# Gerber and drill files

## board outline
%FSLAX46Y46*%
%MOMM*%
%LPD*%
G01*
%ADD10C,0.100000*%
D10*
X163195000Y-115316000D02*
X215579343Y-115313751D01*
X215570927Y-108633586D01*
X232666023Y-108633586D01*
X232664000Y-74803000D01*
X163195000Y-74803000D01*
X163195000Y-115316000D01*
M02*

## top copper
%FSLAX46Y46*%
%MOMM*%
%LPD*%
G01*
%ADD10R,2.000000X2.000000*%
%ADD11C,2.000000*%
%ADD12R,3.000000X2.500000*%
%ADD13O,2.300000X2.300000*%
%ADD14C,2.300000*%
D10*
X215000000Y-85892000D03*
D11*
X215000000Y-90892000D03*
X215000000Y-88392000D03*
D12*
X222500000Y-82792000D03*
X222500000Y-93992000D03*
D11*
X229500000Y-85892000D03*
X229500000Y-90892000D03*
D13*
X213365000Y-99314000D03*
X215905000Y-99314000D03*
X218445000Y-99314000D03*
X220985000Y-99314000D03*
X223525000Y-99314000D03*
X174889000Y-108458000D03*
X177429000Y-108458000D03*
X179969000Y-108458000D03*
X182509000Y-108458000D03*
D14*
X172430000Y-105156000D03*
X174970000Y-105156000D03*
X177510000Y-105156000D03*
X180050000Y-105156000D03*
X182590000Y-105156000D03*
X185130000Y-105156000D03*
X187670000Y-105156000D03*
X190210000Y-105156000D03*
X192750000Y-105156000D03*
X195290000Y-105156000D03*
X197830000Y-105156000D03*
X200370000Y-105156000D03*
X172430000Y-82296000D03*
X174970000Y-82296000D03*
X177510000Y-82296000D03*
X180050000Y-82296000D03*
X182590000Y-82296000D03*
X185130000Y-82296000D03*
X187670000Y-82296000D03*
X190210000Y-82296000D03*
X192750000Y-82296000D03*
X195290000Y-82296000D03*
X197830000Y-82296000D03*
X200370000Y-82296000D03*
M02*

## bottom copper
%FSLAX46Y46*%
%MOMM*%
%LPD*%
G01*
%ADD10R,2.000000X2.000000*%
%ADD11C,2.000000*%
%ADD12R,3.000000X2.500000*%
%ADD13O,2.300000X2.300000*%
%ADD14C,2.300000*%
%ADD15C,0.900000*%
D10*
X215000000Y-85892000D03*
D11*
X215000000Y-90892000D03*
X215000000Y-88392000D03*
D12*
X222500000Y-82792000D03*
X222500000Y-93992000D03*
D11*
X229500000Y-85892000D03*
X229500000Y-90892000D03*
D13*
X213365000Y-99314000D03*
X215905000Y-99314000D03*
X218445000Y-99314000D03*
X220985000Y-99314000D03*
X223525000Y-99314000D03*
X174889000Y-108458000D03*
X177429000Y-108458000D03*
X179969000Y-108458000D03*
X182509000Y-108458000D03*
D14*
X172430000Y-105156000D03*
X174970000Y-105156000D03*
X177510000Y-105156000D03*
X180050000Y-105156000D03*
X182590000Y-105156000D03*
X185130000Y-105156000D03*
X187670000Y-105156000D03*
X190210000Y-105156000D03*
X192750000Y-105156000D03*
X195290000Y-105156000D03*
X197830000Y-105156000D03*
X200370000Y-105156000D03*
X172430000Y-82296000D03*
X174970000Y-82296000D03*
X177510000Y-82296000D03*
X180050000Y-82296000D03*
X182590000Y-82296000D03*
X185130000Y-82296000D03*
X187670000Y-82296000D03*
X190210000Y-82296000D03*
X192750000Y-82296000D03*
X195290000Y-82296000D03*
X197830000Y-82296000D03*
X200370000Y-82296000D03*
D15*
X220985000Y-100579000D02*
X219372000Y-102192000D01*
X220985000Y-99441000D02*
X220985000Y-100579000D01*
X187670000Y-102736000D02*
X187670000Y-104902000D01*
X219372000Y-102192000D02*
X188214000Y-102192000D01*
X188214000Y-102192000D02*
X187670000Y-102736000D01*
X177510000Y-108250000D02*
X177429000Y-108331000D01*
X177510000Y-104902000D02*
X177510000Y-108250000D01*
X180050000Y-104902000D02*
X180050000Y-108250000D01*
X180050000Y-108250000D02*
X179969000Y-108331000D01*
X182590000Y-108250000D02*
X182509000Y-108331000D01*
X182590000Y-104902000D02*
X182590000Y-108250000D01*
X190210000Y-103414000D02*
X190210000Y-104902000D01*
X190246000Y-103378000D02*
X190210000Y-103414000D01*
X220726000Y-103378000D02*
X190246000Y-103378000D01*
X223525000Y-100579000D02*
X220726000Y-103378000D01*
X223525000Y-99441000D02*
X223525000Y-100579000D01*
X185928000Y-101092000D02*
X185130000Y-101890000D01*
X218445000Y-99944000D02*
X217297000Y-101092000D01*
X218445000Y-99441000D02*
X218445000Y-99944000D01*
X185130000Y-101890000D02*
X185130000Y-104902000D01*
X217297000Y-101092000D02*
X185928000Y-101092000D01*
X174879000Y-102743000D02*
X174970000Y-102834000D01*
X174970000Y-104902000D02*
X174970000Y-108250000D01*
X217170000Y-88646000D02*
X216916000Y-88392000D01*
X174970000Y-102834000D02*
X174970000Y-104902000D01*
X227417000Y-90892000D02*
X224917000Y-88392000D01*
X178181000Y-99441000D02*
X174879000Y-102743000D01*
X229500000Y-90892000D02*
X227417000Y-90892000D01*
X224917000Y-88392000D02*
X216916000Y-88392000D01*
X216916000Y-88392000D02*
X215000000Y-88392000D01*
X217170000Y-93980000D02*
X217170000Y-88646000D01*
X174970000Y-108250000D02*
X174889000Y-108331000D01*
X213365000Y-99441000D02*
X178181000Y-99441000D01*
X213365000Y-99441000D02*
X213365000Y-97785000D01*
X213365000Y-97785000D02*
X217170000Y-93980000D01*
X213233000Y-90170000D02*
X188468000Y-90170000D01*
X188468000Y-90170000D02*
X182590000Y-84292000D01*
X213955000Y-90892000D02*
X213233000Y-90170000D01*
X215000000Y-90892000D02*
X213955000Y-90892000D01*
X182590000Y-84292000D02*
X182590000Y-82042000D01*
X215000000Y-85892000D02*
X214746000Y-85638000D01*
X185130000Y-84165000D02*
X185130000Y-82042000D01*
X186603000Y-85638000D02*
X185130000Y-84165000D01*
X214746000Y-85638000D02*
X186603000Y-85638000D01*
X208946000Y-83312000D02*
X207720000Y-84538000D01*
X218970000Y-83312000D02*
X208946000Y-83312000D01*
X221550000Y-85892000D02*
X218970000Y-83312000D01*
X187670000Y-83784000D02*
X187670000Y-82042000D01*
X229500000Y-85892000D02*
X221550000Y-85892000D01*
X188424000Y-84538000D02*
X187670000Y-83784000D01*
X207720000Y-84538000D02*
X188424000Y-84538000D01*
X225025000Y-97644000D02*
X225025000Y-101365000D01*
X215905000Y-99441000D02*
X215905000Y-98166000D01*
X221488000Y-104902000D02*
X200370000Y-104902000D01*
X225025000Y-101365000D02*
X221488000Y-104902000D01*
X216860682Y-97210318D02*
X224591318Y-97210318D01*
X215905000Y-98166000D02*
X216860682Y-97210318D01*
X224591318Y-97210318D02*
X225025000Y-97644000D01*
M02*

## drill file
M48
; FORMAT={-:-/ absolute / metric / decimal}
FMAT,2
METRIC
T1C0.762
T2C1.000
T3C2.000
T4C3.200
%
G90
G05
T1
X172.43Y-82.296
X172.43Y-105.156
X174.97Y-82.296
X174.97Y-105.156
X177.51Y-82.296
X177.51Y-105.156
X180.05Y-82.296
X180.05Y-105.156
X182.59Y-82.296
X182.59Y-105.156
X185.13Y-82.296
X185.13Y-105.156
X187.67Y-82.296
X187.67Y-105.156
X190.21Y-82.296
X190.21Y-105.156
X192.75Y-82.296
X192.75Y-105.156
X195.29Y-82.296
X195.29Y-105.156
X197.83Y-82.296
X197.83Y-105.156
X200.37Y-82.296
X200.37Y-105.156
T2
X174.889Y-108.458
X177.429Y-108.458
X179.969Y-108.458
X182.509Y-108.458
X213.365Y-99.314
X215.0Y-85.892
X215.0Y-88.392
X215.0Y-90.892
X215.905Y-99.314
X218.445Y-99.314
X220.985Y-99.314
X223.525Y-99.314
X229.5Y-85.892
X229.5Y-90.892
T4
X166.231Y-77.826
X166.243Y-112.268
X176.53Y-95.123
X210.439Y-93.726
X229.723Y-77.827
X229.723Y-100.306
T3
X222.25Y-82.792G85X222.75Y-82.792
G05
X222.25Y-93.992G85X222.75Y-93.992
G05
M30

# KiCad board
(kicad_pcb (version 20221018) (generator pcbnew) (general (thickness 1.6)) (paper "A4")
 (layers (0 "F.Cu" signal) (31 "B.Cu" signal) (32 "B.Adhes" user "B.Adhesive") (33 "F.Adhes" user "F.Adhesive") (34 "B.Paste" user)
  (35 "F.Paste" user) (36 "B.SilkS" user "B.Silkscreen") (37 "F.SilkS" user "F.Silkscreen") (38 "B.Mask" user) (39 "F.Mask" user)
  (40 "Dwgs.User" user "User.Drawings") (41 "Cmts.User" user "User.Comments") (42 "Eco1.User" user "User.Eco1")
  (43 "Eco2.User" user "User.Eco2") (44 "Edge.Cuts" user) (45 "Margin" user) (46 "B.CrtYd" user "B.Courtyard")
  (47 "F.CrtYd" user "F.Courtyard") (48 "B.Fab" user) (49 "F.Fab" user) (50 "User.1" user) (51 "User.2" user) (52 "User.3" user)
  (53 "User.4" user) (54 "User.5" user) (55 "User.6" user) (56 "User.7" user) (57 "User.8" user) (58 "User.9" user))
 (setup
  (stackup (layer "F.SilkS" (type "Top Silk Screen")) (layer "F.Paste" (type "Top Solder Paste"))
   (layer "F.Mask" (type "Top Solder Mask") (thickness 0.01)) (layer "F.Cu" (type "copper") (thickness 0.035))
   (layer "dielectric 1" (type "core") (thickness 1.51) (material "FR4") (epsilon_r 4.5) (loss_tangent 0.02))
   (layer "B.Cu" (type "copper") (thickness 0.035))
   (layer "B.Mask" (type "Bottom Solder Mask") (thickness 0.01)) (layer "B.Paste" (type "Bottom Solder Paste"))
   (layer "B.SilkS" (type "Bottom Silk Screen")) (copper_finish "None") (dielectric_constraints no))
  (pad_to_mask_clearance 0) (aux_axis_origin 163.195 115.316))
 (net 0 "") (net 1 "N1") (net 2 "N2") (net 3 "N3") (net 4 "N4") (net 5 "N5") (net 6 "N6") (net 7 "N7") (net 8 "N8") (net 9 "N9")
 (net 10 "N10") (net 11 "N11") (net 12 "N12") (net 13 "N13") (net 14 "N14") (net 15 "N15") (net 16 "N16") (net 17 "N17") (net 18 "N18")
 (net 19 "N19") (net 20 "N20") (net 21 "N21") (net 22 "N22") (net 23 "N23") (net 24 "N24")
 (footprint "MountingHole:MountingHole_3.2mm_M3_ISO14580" (layer "F.Cu") (at 210.439 93.726)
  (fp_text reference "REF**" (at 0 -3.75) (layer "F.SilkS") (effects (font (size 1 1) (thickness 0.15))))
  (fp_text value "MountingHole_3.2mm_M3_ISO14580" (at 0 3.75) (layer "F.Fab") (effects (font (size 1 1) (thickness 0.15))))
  (pad "" np_thru_hole circle (at 0 0) (size 3.2 3.2) (drill 3.2) (layers "*.Cu" "*.Mask")))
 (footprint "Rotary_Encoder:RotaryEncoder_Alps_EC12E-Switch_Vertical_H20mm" (layer "F.Cu") (at 215 85.892)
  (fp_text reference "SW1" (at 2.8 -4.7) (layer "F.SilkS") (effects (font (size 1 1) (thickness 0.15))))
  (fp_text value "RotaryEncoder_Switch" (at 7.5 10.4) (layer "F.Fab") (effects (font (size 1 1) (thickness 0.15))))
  (pad "A" thru_hole rect (at 0 0) (size 2 2) (drill 1) (layers "*.Cu" "*.Mask") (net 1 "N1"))
  (pad "B" thru_hole circle (at 0 5) (size 2 2) (drill 1) (layers "*.Cu" "*.Mask") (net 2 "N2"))
  (pad "C" thru_hole circle (at 0 2.5) (size 2 2) (drill 1) (layers "*.Cu" "*.Mask") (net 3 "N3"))
  (pad "MP" thru_hole rect (at 7.5 -3.1) (size 3 2.5) (drill oval 2.5 2) (layers "*.Cu" "*.Mask"))
  (pad "MP" thru_hole rect (at 7.5 8.1) (size 3 2.5) (drill oval 2.5 2) (layers "*.Cu" "*.Mask"))
  (pad "S1" thru_hole circle (at 14.5 0) (size 2 2) (drill 1) (layers "*.Cu" "*.Mask") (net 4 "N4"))
  (pad "S2" thru_hole circle (at 14.5 5) (size 2 2) (drill 1) (layers "*.Cu" "*.Mask") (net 3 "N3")))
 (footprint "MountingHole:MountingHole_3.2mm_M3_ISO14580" (layer "F.Cu") (at 166.243 112.268)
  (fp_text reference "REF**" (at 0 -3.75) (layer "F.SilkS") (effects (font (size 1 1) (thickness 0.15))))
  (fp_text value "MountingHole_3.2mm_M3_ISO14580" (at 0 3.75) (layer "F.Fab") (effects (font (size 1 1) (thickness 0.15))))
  (pad "" np_thru_hole circle (at 0 0) (size 3.2 3.2) (drill 3.2) (layers "*.Cu" "*.Mask")))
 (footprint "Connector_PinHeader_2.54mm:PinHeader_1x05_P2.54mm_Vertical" (layer "F.Cu") (at 213.365 99.314 90)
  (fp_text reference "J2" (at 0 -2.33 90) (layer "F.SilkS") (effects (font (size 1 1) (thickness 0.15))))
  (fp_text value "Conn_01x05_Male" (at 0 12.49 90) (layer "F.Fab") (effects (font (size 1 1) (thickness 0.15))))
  (pad "1" thru_hole oval (at 0 0 90) (size 2.3 2.3) (drill 1) (layers "*.Cu" "*.Mask") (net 3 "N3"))
  (pad "2" thru_hole oval (at 0 2.54 90) (size 2.3 2.3) (drill 1) (layers "*.Cu" "*.Mask") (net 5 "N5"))
  (pad "3" thru_hole oval (at 0 5.08 90) (size 2.3 2.3) (drill 1) (layers "*.Cu" "*.Mask") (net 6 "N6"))
  (pad "4" thru_hole oval (at 0 7.62 90) (size 2.3 2.3) (drill 1) (layers "*.Cu" "*.Mask") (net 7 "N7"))
  (pad "5" thru_hole oval (at 0 10.16 90) (size 2.3 2.3) (drill 1) (layers "*.Cu" "*.Mask") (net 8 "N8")))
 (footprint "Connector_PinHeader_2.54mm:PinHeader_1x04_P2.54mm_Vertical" (layer "F.Cu") (at 174.889 108.458 90)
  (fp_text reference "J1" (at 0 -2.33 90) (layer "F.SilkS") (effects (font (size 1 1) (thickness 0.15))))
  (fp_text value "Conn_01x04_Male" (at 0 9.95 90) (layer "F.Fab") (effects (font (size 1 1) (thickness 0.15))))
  (pad "1" thru_hole oval (at 0 0 90) (size 2.3 2.3) (drill 1) (layers "*.Cu" "*.Mask") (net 3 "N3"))
  (pad "2" thru_hole oval (at 0 2.54 90) (size 2.3 2.3) (drill 1) (layers "*.Cu" "*.Mask") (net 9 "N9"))
  (pad "3" thru_hole oval (at 0 5.08 90) (size 2.3 2.3) (drill 1) (layers "*.Cu" "*.Mask") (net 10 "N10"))
  (pad "4" thru_hole oval (at 0 7.62 90) (size 2.3 2.3) (drill 1) (layers "*.Cu" "*.Mask") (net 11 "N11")))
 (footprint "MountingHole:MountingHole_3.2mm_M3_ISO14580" (layer "F.Cu") (at 229.743 100.33)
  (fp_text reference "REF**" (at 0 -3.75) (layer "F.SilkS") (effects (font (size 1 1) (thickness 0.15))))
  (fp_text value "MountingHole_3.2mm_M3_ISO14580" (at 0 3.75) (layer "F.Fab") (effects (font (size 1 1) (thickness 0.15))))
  (pad "" np_thru_hole circle (at -0.02 -0.024) (size 3.2 3.2) (drill 3.2) (layers "F&B.Cu" "*.Mask")))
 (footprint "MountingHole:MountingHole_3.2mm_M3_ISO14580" (layer "F.Cu") (at 176.53 95.123)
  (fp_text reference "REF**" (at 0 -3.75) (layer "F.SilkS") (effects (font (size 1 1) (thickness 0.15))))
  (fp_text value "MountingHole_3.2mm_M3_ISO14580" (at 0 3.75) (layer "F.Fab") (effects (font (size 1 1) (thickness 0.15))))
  (pad "" np_thru_hole circle (at 0 0) (size 3.2 3.2) (drill 3.2) (layers "*.Cu" "*.Mask")))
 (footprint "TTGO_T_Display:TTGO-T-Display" (layer "F.Cu") (at 204.688 92.329 -90)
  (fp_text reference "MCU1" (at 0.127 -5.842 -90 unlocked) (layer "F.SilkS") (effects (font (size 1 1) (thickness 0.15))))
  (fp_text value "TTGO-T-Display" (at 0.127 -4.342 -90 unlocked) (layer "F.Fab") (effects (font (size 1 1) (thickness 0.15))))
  (pad "1" thru_hole circle (at 12.827 32.258 270) (size 2.3 2.3) (drill 0.762) (layers "*.Cu" "*.Mask") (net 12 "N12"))
  (pad "2" thru_hole circle (at 12.827 29.718 270) (size 2.3 2.3) (drill 0.762) (layers "*.Cu" "*.Mask") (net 3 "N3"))
  (pad "3" thru_hole circle (at 12.827 27.178 270) (size 2.3 2.3) (drill 0.762) (layers "*.Cu" "*.Mask") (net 9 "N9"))
  (pad "4" thru_hole circle (at 12.827 24.638 270) (size 2.3 2.3) (drill 0.762) (layers "*.Cu" "*.Mask") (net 10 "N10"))
  (pad "5" thru_hole circle (at 12.827 22.098 270) (size 2.3 2.3) (drill 0.762) (layers "*.Cu" "*.Mask") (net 11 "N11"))
  (pad "6" thru_hole circle (at 12.827 19.558 270) (size 2.3 2.3) (drill 0.762) (layers "*.Cu" "*.Mask") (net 6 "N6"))
  (pad "7" thru_hole circle (at 12.827 17.018 270) (size 2.3 2.3) (drill 0.762) (layers "*.Cu" "*.Mask") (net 7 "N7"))
  (pad "8" thru_hole circle (at 12.827 14.478 270) (size 2.3 2.3) (drill 0.762) (layers "*.Cu" "*.Mask") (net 8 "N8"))
  (pad "9" thru_hole circle (at 12.827 11.938 270) (size 2.3 2.3) (drill 0.762) (layers "*.Cu" "*.Mask") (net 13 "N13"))
  (pad "10" thru_hole circle (at 12.827 9.398 270) (size 2.3 2.3) (drill 0.762) (layers "*.Cu" "*.Mask") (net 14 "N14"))
  (pad "11" thru_hole circle (at 12.827 6.858 270) (size 2.3 2.3) (drill 0.762) (layers "*.Cu" "*.Mask") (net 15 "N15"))
  (pad "12" thru_hole circle (at 12.827 4.318 270) (size 2.3 2.3) (drill 0.762) (layers "*.Cu" "*.Mask") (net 5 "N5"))
  (pad "13" thru_hole circle (at -10.033 32.258 270) (size 2.3 2.3) (drill 0.762) (layers "*.Cu" "*.Mask") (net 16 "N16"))
  (pad "14" thru_hole circle (at -10.033 29.718 270) (size 2.3 2.3) (drill 0.762) (layers "*.Cu" "*.Mask") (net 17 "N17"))
  (pad "15" thru_hole circle (at -10.033 27.178 270) (size 2.3 2.3) (drill 0.762) (layers "*.Cu" "*.Mask") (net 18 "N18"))
  (pad "16" thru_hole circle (at -10.033 24.638 270) (size 2.3 2.3) (drill 0.762) (layers "*.Cu" "*.Mask") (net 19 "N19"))
  (pad "17" thru_hole circle (at -10.033 22.098 270) (size 2.3 2.3) (drill 0.762) (layers "*.Cu" "*.Mask") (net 2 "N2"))
  (pad "18" thru_hole circle (at -10.033 19.558 270) (size 2.3 2.3) (drill 0.762) (layers "*.Cu" "*.Mask") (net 1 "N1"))
  (pad "19" thru_hole circle (at -10.033 17.018 270) (size 2.3 2.3) (drill 0.762) (layers "*.Cu" "*.Mask") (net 4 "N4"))
  (pad "20" thru_hole circle (at -10.033 14.478 270) (size 2.3 2.3) (drill 0.762) (layers "*.Cu" "*.Mask") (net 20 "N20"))
  (pad "21" thru_hole circle (at -10.033 11.938 270) (size 2.3 2.3) (drill 0.762) (layers "*.Cu" "*.Mask") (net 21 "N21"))
  (pad "22" thru_hole circle (at -10.033 9.398 270) (size 2.3 2.3) (drill 0.762) (layers "*.Cu" "*.Mask") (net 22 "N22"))
  (pad "23" thru_hole circle (at -10.033 6.858 270) (size 2.3 2.3) (drill 0.762) (layers "*.Cu" "*.Mask") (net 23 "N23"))
  (pad "24" thru_hole circle (at -10.033 4.318 270) (size 2.3 2.3) (drill 0.762) (layers "*.Cu" "*.Mask") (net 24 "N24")))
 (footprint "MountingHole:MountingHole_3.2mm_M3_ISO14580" (layer "F.Cu") (at 166.243 77.849806)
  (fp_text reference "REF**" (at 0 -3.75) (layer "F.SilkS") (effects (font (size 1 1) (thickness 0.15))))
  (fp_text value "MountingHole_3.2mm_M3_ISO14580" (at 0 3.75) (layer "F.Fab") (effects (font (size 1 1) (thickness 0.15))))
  (pad "" np_thru_hole circle (at -0.012 -0.024) (size 3.2 3.2) (drill 3.2) (layers "F&B.Cu" "*.Mask")))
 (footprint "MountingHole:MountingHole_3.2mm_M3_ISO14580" (layer "F.Cu") (at 229.743 77.851)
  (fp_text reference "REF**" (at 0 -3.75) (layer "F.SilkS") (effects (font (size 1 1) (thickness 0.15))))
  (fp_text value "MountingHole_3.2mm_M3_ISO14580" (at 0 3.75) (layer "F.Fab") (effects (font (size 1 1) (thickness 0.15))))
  (pad "" np_thru_hole circle (at -0.02 -0.024) (size 3.2 3.2) (drill 3.2) (layers "F&B.Cu" "*.Mask")))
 (gr_poly
  (pts (xy 163.195 115.316) (xy 215.579343 115.313751) (xy 215.570927 108.633586) (xy 232.666023 108.633586) (xy 232.664 74.803)
   (xy 163.195 74.803))
  (stroke (width 0.1) (type solid)) (fill none) (layer "Edge.Cuts"))
 (segment (start 220.985 100.579) (end 219.372 102.192) (width 0.9) (layer "B.Cu") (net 7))
 (segment (start 220.985 99.441) (end 220.985 100.579) (width 0.9) (layer "B.Cu") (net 7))
 (segment (start 187.67 102.736) (end 187.67 104.902) (width 0.9) (layer "B.Cu") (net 7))
 (segment (start 219.372 102.192) (end 188.214 102.192) (width 0.9) (layer "B.Cu") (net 7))
 (segment (start 188.214 102.192) (end 187.67 102.736) (width 0.9) (layer "B.Cu") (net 7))
 (segment (start 177.51 108.25) (end 177.429 108.331) (width 0.9) (layer "B.Cu") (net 9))
 (segment (start 177.51 104.902) (end 177.51 108.25) (width 0.9) (layer "B.Cu") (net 9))
 (segment (start 180.05 104.902) (end 180.05 108.25) (width 0.9) (layer "B.Cu") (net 10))
 (segment (start 180.05 108.25) (end 179.969 108.331) (width 0.9) (layer "B.Cu") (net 10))
 (segment (start 182.59 108.25) (end 182.509 108.331) (width 0.9) (layer "B.Cu") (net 11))
 (segment (start 182.59 104.902) (end 182.59 108.25) (width 0.9) (layer "B.Cu") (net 11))
 (segment (start 190.21 103.414) (end 190.21 104.902) (width 0.9) (layer "B.Cu") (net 8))
 (segment (start 190.246 103.378) (end 190.21 103.414) (width 0.9) (layer "B.Cu") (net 8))
 (segment (start 220.726 103.378) (end 190.246 103.378) (width 0.9) (layer "B.Cu") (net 8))
 (segment (start 223.525 100.579) (end 220.726 103.378) (width 0.9) (layer "B.Cu") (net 8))
 (segment (start 223.525 99.441) (end 223.525 100.579) (width 0.9) (layer "B.Cu") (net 8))
 (segment (start 185.928 101.092) (end 185.13 101.89) (width 0.9) (layer "B.Cu") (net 6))
 (segment (start 218.445 99.944) (end 217.297 101.092) (width 0.9) (layer "B.Cu") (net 6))
 (segment (start 218.445 99.441) (end 218.445 99.944) (width 0.9) (layer "B.Cu") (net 6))
 (segment (start 185.13 101.89) (end 185.13 104.902) (width 0.9) (layer "B.Cu") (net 6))
 (segment (start 217.297 101.092) (end 185.928 101.092) (width 0.9) (layer "B.Cu") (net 6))
 (segment (start 174.879 102.743) (end 174.97 102.834) (width 0.9) (layer "B.Cu") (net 3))
 (segment (start 174.97 104.902) (end 174.97 108.25) (width 0.9) (layer "B.Cu") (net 3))
 (segment (start 217.17 88.646) (end 216.916 88.392) (width 0.9) (layer "B.Cu") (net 3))
 (segment (start 174.97 102.834) (end 174.97 104.902) (width 0.9) (layer "B.Cu") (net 3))
 (segment (start 227.417 90.892) (end 224.917 88.392) (width 0.9) (layer "B.Cu") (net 3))
 (segment (start 178.181 99.441) (end 174.879 102.743) (width 0.9) (layer "B.Cu") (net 3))
 (segment (start 229.5 90.892) (end 227.417 90.892) (width 0.9) (layer "B.Cu") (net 3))
 (segment (start 224.917 88.392) (end 216.916 88.392) (width 0.9) (layer "B.Cu") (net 3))
 (segment (start 216.916 88.392) (end 215 88.392) (width 0.9) (layer "B.Cu") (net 3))
 (segment (start 217.17 93.98) (end 217.17 88.646) (width 0.9) (layer "B.Cu") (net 3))
 (segment (start 174.97 108.25) (end 174.889 108.331) (width 0.9) (layer "B.Cu") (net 3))
 (segment (start 213.365 99.441) (end 178.181 99.441) (width 0.9) (layer "B.Cu") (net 3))
 (segment (start 213.365 99.441) (end 213.365 97.785) (width 0.9) (layer "B.Cu") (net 3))
 (segment (start 213.365 97.785) (end 217.17 93.98) (width 0.9) (layer "B.Cu") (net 3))
 (segment (start 213.233 90.17) (end 188.468 90.17) (width 0.9) (layer "B.Cu") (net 2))
 (segment (start 188.468 90.17) (end 182.59 84.292) (width 0.9) (layer "B.Cu") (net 2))
 (segment (start 213.955 90.892) (end 213.233 90.17) (width 0.9) (layer "B.Cu") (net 2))
 (segment (start 215 90.892) (end 213.955 90.892) (width 0.9) (layer "B.Cu") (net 2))
 (segment (start 182.59 84.292) (end 182.59 82.042) (width 0.9) (layer "B.Cu") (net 2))
 (segment (start 215 85.892) (end 214.746 85.638) (width 0.9) (layer "B.Cu") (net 1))
 (segment (start 185.13 84.165) (end 185.13 82.042) (width 0.9) (layer "B.Cu") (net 1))
 (segment (start 186.603 85.638) (end 185.13 84.165) (width 0.9) (layer "B.Cu") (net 1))
 (segment (start 214.746 85.638) (end 186.603 85.638) (width 0.9) (layer "B.Cu") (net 1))
 (segment (start 208.946 83.312) (end 207.72 84.538) (width 0.9) (layer "B.Cu") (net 4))
 (segment (start 218.97 83.312) (end 208.946 83.312) (width 0.9) (layer "B.Cu") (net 4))
 (segment (start 221.55 85.892) (end 218.97 83.312) (width 0.9) (layer "B.Cu") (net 4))
 (segment (start 187.67 83.784) (end 187.67 82.042) (width 0.9) (layer "B.Cu") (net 4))
 (segment (start 229.5 85.892) (end 221.55 85.892) (width 0.9) (layer "B.Cu") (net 4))
 (segment (start 188.424 84.538) (end 187.67 83.784) (width 0.9) (layer "B.Cu") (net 4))
 (segment (start 207.72 84.538) (end 188.424 84.538) (width 0.9) (layer "B.Cu") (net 4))
 (segment (start 225.025 97.644) (end 225.025 101.365) (width 0.9) (layer "B.Cu") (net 5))
 (segment (start 215.905 99.441) (end 215.905 98.166) (width 0.9) (layer "B.Cu") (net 5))
 (segment (start 221.488 104.902) (end 200.37 104.902) (width 0.9) (layer "B.Cu") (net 5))
 (segment (start 225.025 101.365) (end 221.488 104.902) (width 0.9) (layer "B.Cu") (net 5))
 (segment (start 216.860682 97.210318) (end 224.591318 97.210318) (width 0.9) (layer "B.Cu") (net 5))
 (segment (start 215.905 98.166) (end 216.860682 97.210318) (width 0.9) (layer "B.Cu") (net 5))
 (segment (start 224.591318 97.210318) (end 225.025 97.644) (width 0.9) (layer "B.Cu") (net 5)))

